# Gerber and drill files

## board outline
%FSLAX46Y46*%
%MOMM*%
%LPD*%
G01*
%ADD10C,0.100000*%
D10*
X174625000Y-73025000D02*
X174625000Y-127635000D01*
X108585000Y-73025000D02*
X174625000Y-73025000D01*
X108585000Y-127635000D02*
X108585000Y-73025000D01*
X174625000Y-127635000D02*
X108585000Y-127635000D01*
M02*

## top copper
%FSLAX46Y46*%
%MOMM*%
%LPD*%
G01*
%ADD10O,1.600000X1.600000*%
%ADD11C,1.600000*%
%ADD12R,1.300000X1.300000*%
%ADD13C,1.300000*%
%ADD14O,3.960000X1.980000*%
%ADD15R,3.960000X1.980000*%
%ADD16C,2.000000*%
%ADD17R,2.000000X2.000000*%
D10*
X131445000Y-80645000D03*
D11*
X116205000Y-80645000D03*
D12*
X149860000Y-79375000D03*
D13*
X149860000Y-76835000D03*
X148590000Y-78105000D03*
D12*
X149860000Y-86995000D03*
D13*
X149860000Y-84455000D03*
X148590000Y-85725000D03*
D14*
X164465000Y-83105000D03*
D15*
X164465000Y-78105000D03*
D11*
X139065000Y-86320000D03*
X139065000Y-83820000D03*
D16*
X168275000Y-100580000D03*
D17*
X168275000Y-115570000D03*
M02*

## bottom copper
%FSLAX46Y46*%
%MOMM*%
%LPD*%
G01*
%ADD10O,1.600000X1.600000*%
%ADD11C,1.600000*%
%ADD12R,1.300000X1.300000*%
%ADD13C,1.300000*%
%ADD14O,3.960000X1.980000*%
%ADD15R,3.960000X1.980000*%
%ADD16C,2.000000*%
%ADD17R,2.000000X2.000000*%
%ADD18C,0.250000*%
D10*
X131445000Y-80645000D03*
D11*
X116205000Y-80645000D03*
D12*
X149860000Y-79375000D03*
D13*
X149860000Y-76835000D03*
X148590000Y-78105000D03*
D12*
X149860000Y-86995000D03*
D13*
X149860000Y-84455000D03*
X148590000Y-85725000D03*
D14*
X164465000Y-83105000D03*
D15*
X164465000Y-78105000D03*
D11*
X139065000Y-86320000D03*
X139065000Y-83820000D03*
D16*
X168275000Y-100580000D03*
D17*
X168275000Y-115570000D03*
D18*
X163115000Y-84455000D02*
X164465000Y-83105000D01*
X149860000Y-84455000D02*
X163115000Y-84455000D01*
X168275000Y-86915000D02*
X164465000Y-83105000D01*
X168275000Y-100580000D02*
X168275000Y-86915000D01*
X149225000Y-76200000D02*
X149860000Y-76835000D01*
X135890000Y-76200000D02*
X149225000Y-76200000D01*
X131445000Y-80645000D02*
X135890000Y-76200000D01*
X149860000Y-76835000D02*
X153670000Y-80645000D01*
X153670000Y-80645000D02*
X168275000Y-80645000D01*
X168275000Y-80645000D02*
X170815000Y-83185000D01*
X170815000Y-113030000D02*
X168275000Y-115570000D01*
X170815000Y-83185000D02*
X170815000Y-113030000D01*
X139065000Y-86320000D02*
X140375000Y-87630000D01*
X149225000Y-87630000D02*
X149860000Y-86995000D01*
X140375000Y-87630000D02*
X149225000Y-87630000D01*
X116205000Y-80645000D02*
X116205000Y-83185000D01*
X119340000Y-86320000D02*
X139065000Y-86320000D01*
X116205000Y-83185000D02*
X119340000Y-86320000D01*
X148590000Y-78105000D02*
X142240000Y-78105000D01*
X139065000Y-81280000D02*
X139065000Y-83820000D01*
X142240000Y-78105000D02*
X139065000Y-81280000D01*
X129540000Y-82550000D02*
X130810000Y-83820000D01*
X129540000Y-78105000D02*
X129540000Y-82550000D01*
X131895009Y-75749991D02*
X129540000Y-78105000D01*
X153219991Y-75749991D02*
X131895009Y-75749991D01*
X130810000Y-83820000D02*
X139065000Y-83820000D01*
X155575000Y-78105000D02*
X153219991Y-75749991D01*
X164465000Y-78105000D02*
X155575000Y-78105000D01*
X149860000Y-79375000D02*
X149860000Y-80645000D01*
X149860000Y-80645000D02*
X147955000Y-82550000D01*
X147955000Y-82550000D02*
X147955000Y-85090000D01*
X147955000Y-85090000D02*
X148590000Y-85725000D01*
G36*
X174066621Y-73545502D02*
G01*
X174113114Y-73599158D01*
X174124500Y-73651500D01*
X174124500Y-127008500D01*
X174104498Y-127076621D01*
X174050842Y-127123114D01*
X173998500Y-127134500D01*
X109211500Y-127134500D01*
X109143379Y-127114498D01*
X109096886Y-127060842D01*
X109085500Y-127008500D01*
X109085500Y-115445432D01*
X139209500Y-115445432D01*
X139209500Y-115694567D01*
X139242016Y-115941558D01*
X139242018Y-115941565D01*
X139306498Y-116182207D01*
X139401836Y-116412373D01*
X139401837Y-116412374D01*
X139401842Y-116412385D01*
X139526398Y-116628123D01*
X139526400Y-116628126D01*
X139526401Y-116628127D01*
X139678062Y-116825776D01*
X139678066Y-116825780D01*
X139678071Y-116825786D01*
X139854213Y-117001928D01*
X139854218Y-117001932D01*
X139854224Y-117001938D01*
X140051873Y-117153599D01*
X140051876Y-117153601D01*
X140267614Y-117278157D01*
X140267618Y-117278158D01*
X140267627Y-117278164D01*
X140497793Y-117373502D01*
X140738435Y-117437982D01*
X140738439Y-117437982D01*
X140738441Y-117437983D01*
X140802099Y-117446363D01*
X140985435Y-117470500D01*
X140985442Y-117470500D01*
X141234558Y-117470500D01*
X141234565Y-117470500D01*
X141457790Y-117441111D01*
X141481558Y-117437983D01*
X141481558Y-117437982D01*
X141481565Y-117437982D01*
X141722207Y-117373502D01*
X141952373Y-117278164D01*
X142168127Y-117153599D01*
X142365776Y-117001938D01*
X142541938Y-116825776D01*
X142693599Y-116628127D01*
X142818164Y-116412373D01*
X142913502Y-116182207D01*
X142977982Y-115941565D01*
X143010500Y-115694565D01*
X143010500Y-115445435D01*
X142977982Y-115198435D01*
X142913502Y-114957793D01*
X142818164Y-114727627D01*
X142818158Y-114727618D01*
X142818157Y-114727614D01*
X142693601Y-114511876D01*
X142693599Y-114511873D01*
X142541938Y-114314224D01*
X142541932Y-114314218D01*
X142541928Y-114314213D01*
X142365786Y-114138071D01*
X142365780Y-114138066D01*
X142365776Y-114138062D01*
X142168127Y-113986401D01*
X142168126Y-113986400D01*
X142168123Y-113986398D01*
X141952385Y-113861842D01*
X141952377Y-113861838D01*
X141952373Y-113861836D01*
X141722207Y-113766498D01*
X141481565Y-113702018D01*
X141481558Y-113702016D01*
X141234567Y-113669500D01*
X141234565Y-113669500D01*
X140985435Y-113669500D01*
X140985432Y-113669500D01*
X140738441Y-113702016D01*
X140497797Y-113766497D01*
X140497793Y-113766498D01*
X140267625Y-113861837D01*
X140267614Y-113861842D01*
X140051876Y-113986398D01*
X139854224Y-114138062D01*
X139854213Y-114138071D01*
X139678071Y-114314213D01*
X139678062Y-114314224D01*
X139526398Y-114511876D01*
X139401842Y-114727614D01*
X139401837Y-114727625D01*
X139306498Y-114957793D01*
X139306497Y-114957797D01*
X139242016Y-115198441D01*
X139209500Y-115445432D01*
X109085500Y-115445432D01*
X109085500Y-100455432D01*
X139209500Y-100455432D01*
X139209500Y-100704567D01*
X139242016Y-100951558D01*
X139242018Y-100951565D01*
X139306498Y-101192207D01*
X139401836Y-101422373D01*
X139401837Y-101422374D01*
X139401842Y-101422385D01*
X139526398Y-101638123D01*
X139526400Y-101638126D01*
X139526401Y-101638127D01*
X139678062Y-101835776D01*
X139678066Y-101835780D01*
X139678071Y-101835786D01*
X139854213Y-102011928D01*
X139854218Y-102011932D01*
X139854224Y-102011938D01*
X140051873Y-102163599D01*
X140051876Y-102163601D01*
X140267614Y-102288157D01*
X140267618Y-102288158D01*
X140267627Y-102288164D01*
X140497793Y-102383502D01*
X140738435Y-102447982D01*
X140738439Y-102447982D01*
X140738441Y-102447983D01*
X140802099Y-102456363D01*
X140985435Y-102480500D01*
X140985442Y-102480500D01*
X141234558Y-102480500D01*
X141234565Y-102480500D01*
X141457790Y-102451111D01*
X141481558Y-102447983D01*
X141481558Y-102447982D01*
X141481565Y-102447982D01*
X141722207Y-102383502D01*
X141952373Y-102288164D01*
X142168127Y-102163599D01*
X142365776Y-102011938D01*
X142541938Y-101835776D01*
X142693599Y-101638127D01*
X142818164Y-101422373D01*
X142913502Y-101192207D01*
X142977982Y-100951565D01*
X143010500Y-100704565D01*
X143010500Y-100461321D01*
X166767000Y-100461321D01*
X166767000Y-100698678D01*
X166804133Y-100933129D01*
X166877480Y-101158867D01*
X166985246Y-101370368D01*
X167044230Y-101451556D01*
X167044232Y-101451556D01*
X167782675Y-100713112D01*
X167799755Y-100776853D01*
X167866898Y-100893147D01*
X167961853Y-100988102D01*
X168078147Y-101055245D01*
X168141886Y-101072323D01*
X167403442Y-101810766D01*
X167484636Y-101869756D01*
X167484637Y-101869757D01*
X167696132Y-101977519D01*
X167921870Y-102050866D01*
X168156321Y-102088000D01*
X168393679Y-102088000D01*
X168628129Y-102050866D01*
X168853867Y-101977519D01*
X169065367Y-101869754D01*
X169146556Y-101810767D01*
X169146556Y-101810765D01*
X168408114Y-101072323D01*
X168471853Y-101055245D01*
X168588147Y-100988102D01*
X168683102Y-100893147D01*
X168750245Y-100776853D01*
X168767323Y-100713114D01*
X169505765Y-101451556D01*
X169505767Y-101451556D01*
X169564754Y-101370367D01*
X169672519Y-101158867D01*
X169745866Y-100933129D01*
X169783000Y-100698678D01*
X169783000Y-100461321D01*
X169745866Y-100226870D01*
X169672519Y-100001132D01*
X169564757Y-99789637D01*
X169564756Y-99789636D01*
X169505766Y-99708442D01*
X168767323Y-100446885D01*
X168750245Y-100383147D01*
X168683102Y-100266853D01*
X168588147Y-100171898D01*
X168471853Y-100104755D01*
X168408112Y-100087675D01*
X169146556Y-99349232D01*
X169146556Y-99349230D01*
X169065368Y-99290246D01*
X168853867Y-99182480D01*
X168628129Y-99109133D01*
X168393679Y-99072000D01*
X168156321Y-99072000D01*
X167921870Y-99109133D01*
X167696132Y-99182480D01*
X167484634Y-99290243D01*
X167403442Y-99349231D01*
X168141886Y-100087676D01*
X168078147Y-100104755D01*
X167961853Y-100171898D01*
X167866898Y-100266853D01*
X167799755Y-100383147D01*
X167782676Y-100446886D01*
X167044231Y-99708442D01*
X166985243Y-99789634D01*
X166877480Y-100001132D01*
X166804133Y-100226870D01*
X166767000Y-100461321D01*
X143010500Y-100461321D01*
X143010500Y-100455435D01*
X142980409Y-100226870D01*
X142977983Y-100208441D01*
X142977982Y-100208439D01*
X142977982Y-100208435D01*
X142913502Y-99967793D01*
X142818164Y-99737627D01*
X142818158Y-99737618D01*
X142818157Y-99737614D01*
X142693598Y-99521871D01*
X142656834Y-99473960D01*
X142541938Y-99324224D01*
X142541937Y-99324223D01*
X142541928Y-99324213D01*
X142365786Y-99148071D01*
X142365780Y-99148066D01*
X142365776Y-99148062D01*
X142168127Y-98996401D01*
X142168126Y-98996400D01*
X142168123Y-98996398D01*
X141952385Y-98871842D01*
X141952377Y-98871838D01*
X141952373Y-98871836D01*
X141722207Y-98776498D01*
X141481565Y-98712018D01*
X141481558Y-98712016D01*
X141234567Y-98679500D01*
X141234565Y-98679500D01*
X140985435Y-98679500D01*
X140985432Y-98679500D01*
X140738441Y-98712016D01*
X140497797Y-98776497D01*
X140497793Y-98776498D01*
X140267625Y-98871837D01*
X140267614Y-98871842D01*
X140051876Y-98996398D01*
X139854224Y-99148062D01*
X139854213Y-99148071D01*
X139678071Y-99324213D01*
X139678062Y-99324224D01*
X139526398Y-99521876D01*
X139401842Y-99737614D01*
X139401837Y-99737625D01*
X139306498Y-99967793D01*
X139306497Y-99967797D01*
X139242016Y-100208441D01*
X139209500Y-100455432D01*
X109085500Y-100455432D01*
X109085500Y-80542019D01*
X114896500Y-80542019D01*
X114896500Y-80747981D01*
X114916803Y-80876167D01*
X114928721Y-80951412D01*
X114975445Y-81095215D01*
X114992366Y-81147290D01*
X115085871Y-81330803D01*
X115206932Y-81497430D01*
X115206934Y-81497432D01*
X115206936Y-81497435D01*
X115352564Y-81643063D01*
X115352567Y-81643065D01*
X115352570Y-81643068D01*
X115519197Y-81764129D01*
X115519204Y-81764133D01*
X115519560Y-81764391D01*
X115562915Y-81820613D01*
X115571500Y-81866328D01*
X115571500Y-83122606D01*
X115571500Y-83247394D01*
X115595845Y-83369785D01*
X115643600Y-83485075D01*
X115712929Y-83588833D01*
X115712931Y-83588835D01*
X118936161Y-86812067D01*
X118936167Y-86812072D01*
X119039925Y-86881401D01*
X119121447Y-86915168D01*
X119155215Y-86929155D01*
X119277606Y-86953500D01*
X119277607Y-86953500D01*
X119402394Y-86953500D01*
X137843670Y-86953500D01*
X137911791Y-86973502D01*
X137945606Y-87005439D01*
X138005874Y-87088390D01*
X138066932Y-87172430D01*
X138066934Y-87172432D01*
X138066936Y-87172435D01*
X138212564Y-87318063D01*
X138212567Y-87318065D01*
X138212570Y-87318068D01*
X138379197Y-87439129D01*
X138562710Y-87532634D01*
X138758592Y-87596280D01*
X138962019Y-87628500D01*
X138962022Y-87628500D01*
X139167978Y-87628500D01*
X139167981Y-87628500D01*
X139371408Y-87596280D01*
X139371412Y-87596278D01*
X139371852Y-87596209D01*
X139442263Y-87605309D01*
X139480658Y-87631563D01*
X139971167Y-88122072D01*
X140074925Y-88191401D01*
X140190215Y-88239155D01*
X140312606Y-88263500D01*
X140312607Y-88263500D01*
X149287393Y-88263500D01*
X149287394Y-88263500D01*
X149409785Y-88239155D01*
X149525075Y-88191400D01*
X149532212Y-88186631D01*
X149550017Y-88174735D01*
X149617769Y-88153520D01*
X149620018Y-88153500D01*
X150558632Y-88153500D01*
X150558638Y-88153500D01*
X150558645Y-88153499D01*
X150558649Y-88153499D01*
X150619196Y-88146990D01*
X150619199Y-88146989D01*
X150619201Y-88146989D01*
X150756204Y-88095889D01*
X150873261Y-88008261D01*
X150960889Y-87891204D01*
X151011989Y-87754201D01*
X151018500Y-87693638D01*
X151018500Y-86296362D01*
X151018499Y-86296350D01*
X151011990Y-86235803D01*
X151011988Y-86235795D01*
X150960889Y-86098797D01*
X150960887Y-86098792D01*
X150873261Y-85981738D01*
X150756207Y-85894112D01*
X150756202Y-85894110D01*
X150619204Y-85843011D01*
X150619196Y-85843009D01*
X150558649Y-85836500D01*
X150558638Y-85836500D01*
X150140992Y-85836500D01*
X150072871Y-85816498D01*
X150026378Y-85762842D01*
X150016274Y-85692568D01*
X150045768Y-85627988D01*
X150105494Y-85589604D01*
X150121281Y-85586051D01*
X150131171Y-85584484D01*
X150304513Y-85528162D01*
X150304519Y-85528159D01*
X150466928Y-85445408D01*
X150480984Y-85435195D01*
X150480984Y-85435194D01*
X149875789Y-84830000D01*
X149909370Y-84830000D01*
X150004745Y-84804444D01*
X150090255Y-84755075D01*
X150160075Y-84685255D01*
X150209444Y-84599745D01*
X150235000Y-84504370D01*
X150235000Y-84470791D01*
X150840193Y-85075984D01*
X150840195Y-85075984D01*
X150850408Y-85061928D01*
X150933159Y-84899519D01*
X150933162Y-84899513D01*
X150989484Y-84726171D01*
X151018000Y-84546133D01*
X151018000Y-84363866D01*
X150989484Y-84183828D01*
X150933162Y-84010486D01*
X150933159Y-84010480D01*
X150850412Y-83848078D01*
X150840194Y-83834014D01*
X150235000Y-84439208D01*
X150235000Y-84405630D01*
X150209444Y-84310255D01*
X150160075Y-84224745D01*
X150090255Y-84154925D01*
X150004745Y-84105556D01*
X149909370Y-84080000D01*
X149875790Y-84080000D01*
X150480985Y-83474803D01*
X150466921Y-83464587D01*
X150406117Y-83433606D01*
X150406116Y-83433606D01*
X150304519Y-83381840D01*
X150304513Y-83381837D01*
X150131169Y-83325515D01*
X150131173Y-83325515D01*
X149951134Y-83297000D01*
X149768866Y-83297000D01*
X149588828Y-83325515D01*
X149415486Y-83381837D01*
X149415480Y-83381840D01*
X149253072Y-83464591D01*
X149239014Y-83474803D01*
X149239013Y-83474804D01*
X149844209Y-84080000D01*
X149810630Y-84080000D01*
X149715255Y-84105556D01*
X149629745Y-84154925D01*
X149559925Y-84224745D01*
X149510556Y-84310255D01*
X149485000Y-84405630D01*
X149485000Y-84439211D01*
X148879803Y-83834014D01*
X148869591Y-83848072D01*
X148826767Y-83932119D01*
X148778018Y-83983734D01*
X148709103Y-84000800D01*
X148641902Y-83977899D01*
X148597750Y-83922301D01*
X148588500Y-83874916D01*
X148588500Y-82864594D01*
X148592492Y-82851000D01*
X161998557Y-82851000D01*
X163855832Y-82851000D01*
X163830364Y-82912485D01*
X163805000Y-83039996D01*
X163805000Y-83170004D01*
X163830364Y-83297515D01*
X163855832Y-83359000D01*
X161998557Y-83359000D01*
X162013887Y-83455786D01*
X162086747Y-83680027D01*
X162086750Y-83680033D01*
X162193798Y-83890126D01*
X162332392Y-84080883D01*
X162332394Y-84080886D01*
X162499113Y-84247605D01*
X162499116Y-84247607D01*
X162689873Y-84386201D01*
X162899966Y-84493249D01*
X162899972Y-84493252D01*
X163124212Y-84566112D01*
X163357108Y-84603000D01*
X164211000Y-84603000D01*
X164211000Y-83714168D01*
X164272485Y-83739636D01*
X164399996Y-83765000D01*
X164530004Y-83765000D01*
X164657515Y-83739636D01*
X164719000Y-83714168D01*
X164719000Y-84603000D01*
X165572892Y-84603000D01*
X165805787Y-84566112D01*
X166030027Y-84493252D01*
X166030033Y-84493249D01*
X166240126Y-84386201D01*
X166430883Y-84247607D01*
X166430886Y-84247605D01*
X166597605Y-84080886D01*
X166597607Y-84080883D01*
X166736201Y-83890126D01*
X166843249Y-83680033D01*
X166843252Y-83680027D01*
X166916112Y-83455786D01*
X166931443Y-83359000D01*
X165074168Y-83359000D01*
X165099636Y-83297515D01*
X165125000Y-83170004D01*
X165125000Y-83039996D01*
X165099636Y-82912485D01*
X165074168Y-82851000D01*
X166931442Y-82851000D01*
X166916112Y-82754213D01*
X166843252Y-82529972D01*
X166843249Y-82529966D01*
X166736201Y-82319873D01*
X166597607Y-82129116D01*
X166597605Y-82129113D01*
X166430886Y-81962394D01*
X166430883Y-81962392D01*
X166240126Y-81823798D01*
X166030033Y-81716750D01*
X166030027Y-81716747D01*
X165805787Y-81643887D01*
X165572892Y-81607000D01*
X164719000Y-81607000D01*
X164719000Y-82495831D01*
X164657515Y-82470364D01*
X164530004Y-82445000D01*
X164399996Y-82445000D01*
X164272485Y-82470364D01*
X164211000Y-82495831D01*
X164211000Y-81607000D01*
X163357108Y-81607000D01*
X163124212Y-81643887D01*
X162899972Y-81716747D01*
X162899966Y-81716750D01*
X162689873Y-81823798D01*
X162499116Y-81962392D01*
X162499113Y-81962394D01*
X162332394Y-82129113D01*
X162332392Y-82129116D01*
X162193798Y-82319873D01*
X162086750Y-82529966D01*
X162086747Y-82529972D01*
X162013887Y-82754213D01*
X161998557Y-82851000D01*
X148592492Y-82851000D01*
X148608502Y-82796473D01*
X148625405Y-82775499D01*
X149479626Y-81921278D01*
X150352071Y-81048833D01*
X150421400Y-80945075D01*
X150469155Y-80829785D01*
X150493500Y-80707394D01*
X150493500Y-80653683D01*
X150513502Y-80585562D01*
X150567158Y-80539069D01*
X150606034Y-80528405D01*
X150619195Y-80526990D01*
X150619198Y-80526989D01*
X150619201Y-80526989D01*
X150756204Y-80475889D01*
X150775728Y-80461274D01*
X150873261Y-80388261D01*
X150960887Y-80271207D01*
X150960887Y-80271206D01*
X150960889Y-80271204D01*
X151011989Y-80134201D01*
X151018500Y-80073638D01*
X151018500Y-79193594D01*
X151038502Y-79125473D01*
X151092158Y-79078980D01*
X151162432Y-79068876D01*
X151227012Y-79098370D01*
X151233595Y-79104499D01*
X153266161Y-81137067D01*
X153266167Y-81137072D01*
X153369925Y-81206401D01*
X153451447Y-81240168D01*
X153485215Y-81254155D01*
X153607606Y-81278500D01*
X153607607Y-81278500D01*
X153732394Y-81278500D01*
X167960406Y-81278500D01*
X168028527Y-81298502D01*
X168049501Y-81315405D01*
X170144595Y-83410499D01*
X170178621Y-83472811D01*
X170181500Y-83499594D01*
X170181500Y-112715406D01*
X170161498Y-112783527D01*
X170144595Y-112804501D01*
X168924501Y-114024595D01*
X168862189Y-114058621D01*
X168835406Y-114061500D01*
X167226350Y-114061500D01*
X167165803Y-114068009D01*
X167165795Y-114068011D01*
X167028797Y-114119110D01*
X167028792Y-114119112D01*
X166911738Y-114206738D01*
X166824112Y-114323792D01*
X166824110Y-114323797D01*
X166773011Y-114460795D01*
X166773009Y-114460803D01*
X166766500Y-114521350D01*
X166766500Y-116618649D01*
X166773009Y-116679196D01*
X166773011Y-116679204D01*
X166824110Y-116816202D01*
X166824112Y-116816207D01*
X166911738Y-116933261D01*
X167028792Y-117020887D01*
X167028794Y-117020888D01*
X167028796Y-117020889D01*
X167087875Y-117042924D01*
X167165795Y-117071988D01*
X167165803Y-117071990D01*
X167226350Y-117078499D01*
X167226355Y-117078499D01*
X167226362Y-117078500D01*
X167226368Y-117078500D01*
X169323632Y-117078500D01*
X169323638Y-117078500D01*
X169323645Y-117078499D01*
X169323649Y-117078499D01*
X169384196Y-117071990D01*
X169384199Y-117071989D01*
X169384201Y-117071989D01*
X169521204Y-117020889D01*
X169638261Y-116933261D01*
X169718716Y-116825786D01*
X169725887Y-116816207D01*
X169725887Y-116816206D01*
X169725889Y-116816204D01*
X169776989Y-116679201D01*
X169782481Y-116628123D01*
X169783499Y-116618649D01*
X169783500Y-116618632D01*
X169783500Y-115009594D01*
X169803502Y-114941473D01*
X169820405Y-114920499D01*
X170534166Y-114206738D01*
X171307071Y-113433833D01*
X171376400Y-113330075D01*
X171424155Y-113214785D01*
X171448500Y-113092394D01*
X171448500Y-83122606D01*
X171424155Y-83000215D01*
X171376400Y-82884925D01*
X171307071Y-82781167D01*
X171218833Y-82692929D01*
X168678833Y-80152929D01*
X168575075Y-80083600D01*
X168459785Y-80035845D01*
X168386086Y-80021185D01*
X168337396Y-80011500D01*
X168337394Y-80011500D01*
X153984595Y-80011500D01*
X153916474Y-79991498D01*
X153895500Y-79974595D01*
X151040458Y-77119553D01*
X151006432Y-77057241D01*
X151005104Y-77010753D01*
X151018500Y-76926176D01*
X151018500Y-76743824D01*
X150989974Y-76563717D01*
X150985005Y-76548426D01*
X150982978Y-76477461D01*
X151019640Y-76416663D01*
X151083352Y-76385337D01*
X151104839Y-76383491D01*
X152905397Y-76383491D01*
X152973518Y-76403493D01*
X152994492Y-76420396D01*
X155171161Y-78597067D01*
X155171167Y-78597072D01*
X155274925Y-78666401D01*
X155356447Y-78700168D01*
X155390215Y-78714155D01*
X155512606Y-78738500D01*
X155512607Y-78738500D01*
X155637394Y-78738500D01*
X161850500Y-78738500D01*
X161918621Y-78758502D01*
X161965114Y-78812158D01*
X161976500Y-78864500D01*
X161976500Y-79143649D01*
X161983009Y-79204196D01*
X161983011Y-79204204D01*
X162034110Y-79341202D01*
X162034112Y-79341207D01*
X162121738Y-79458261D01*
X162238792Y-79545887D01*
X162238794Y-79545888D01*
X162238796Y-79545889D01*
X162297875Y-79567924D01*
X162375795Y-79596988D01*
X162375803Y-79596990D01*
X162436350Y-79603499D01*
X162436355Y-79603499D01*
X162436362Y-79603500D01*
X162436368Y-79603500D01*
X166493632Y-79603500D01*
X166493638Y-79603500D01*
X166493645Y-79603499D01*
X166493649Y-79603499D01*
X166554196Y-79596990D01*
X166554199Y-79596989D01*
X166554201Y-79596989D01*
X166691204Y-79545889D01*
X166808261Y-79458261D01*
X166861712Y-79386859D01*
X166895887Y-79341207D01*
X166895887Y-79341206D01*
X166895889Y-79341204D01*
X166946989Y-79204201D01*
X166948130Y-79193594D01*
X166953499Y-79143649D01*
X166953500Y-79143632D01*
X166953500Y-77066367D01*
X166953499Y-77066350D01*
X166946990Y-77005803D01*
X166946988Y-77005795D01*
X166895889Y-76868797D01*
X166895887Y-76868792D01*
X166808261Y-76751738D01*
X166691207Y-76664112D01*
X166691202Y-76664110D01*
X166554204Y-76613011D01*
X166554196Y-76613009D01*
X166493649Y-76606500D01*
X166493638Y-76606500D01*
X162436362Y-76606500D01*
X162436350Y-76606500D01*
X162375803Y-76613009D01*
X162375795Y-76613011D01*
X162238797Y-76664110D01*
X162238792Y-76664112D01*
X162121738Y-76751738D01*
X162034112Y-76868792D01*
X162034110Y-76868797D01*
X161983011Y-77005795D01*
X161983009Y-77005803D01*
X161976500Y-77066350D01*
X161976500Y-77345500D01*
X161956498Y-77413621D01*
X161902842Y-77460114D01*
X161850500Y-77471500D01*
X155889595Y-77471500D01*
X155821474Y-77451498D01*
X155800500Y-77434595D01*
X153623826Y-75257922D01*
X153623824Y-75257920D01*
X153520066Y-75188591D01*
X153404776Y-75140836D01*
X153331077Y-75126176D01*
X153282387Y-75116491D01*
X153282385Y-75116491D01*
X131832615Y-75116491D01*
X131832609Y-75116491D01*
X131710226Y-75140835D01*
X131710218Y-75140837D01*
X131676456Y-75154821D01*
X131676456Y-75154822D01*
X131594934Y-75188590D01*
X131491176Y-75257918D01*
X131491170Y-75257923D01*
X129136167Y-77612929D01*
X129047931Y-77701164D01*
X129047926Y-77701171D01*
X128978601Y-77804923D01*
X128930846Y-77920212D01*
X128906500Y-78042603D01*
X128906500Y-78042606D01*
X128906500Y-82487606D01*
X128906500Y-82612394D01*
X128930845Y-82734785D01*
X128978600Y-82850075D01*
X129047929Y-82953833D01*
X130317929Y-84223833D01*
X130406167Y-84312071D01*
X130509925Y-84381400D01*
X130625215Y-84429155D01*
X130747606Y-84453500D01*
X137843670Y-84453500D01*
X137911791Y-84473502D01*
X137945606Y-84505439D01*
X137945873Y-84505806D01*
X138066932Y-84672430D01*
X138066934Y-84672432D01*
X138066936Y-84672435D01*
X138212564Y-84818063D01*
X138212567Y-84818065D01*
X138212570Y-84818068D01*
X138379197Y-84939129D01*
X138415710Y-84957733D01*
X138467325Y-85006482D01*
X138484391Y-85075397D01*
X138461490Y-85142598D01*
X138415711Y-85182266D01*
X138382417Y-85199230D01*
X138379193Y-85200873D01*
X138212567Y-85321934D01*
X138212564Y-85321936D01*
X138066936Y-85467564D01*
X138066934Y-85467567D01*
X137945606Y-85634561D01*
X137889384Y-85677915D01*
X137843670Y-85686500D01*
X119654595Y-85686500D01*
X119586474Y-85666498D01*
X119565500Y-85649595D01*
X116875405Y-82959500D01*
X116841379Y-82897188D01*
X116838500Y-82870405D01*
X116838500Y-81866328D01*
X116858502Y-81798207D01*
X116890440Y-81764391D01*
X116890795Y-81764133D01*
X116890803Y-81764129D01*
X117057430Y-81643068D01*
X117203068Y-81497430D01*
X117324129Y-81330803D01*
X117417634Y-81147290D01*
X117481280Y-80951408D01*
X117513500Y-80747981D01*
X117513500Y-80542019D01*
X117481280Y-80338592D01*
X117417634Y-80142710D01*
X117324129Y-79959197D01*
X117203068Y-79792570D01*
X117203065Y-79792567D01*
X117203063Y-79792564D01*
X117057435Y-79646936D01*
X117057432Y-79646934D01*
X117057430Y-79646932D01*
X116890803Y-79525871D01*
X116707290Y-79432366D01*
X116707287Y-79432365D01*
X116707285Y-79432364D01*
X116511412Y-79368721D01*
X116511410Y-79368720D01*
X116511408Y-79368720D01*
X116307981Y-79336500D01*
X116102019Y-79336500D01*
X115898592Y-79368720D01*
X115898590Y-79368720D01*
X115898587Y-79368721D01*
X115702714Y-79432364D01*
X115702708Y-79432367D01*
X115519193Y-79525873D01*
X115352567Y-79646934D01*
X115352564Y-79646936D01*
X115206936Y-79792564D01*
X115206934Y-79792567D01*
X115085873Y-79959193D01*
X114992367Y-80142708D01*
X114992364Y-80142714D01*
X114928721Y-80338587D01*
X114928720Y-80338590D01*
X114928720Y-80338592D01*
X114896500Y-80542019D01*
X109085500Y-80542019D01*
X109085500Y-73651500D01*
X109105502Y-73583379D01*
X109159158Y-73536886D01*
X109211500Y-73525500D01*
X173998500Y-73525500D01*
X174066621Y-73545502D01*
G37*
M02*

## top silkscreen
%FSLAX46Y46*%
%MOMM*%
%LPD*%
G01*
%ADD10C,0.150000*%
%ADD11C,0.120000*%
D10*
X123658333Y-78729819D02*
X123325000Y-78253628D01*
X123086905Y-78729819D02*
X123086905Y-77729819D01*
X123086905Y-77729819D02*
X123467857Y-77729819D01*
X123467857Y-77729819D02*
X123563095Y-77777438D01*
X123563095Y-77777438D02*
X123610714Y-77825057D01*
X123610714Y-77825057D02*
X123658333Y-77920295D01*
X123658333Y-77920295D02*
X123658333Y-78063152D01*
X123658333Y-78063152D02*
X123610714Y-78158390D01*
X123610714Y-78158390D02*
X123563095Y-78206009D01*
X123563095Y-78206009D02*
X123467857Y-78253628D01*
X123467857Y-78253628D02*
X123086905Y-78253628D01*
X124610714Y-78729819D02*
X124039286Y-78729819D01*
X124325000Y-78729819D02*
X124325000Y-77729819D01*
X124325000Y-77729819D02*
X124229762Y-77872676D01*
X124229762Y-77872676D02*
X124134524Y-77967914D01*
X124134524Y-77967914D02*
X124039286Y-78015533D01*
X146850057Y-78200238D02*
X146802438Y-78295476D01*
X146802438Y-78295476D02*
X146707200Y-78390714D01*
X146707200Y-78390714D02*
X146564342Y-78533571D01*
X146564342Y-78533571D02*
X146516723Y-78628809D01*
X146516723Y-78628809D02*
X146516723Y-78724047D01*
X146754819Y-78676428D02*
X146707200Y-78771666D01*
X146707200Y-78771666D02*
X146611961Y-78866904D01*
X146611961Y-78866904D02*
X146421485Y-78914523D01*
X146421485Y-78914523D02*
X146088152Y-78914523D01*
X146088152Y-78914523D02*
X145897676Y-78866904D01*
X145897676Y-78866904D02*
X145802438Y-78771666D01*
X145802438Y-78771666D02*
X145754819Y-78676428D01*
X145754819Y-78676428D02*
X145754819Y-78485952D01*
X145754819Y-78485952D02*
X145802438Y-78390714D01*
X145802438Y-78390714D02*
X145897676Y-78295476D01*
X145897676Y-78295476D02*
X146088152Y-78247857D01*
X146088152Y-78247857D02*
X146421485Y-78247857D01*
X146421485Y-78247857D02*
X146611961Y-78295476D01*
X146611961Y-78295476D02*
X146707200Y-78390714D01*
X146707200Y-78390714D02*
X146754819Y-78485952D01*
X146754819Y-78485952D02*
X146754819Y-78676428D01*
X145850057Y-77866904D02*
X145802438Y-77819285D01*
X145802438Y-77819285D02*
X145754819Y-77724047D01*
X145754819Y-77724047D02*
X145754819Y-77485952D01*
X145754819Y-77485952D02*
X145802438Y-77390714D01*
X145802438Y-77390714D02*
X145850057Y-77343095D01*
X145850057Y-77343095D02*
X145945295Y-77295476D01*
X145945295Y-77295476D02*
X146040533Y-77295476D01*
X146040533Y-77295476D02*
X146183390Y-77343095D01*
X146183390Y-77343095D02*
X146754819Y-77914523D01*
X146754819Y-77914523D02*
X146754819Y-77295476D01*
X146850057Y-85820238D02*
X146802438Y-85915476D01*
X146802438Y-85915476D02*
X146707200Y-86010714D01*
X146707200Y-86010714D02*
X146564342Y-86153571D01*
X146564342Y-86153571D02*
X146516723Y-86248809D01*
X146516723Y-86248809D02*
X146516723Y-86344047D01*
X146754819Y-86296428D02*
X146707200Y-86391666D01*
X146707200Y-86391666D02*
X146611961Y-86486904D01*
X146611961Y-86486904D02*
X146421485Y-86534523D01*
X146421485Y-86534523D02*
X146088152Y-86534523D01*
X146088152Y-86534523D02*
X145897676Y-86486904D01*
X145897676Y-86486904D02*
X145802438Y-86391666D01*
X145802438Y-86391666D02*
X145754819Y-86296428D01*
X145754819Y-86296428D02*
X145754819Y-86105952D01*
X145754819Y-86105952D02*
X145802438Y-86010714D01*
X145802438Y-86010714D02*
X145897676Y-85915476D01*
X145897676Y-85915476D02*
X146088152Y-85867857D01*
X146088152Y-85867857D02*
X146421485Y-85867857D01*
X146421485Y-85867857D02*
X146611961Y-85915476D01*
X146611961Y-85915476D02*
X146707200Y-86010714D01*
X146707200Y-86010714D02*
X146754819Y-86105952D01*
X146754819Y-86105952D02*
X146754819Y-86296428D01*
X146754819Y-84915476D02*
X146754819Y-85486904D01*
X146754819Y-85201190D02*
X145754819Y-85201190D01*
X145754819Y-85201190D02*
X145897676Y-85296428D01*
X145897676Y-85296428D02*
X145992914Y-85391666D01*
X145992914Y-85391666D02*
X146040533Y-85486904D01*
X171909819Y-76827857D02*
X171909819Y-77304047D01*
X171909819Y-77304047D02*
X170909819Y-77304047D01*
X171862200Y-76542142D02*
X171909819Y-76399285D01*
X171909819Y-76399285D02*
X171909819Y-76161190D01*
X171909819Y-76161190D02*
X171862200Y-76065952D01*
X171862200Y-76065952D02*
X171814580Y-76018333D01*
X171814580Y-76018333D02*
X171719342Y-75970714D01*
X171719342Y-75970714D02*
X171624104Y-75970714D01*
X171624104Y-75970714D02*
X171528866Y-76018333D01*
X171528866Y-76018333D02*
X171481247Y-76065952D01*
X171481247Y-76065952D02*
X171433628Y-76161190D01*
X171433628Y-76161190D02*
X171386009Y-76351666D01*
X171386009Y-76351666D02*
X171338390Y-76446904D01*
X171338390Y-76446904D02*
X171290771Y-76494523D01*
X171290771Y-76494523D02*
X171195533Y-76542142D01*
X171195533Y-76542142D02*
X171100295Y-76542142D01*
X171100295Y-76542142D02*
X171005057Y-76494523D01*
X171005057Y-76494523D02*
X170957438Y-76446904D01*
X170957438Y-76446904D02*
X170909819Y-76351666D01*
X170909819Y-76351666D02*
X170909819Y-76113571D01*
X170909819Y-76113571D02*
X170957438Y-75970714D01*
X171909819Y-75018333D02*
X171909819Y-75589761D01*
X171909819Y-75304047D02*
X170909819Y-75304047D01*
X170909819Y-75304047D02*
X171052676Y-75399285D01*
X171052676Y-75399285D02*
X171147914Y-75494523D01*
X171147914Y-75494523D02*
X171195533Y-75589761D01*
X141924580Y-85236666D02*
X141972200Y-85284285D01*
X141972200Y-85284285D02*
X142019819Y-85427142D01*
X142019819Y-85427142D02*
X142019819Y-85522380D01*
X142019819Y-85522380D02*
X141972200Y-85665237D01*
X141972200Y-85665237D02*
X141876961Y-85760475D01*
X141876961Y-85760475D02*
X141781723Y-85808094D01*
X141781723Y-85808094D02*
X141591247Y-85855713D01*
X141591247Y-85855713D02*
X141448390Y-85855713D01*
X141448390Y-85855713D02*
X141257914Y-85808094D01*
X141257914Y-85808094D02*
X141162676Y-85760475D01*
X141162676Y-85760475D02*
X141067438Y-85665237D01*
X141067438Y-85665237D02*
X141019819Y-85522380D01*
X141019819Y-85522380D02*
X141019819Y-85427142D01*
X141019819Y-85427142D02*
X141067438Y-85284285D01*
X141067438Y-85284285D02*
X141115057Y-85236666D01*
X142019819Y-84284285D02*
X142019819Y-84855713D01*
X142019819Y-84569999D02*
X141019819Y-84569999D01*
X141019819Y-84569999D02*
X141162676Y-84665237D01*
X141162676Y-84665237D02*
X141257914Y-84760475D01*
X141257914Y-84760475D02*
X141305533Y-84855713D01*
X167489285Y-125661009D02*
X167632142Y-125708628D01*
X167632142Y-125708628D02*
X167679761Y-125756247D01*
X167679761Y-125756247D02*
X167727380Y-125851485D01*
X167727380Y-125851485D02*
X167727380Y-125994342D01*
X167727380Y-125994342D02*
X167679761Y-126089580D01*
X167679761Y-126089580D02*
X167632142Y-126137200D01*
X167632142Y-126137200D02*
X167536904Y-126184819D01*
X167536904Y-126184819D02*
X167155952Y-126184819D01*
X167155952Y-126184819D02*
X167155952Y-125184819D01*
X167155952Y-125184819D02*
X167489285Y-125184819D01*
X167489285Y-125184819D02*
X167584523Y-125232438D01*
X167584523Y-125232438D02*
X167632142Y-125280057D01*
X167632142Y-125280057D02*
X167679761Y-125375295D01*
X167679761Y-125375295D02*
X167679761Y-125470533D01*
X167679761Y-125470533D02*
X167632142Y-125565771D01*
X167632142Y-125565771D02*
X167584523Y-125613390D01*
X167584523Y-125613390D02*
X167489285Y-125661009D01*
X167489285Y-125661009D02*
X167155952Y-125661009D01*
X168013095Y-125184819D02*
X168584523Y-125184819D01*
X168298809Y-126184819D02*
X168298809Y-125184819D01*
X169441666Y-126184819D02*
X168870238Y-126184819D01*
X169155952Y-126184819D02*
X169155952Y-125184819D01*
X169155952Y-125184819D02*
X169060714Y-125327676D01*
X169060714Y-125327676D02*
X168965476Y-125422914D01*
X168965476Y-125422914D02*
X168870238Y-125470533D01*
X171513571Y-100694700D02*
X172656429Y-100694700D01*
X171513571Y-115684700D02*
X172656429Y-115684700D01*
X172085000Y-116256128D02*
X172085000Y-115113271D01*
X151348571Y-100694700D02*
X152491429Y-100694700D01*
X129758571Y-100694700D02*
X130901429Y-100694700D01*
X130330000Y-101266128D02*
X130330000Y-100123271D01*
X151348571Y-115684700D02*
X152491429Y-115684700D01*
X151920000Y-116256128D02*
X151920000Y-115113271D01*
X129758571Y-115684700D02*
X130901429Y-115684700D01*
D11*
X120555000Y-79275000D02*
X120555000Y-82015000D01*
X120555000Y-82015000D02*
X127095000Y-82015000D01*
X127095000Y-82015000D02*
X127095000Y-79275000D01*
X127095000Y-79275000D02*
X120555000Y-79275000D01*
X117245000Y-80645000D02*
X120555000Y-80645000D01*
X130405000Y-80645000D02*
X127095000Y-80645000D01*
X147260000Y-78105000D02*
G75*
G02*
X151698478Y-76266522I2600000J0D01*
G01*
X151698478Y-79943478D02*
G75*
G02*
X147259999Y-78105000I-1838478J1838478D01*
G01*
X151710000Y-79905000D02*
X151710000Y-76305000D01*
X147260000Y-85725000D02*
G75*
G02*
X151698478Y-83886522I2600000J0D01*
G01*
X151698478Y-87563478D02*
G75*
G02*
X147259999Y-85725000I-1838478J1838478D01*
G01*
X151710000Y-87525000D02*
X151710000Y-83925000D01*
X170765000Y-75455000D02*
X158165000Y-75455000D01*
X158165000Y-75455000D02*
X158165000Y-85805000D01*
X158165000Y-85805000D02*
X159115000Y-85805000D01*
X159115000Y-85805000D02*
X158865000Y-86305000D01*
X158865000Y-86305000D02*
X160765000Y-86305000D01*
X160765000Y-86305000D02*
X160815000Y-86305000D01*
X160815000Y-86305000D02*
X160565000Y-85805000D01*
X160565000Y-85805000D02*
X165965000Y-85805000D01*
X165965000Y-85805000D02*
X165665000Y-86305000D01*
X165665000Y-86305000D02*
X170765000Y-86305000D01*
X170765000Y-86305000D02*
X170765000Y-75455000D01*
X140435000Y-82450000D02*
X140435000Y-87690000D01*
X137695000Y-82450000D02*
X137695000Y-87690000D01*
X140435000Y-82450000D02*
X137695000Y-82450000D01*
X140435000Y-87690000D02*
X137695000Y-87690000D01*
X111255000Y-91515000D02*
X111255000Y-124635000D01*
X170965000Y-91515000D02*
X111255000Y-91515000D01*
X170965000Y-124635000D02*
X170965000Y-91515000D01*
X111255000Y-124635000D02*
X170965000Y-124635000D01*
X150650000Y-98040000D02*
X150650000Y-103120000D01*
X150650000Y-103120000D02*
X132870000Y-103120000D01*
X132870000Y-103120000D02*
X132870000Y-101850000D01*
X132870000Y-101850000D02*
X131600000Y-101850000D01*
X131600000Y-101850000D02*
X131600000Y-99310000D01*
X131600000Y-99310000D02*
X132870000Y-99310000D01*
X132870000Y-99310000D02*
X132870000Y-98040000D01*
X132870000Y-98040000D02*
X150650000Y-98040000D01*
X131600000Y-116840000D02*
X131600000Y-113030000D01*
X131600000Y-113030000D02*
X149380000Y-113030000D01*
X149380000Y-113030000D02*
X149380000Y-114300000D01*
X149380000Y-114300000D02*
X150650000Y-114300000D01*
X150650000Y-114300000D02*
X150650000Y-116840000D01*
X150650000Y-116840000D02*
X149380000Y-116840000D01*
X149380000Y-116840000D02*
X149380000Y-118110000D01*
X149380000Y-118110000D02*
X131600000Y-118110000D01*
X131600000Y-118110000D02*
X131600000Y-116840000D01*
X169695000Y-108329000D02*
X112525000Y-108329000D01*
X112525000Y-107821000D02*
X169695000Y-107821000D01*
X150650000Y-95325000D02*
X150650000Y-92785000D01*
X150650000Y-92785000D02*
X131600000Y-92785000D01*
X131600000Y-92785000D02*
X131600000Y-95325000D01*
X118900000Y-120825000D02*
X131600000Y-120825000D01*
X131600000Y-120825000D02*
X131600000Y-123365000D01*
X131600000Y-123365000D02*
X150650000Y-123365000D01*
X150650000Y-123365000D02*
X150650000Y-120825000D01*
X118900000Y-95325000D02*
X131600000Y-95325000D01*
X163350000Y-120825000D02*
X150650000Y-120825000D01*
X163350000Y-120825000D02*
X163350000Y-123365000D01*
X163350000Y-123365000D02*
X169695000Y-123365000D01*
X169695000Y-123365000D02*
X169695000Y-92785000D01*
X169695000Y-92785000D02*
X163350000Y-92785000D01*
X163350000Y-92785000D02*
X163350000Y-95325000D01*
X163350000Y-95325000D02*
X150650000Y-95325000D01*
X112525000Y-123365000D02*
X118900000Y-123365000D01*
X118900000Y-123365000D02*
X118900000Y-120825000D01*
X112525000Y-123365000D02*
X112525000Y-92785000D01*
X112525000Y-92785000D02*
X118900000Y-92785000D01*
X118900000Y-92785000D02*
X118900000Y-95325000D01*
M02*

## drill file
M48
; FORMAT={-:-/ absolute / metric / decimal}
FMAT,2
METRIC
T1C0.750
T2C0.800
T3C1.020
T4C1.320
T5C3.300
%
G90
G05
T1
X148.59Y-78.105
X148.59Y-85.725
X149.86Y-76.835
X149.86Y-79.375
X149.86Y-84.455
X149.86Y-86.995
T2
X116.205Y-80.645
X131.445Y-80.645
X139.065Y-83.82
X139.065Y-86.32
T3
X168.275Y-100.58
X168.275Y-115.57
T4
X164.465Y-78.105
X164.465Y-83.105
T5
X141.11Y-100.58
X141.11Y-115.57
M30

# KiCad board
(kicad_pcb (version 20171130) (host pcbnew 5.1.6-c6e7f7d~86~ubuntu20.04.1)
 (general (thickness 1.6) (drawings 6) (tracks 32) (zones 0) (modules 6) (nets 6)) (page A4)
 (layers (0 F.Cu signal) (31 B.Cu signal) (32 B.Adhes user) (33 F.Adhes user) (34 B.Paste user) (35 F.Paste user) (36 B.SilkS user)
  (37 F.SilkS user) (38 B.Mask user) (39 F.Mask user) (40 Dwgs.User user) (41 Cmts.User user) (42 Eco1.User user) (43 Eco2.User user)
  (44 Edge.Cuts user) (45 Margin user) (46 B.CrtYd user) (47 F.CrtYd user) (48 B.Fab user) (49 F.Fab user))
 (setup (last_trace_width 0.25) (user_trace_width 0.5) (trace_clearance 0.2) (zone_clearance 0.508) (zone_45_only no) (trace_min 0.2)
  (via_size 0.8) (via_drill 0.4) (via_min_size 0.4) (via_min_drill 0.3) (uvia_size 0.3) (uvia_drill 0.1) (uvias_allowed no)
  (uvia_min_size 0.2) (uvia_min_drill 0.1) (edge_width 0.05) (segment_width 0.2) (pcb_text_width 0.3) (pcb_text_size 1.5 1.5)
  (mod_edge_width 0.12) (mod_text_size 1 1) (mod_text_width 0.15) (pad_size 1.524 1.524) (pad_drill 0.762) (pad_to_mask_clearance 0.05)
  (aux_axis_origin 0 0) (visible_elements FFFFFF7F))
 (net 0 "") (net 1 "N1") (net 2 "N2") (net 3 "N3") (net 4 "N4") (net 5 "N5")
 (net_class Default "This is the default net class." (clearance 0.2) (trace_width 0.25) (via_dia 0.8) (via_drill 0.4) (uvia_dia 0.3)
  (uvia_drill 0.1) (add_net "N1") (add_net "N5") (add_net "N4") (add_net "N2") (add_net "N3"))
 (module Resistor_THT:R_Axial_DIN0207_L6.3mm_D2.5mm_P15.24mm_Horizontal (layer F.Cu) (at 116.205 80.645)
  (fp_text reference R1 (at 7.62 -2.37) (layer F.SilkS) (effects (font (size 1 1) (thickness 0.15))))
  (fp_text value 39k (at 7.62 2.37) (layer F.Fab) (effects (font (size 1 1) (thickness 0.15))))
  (fp_line (start 4.35 -1.37) (end 4.35 1.37) (layer F.SilkS) (width 0.12))
  (fp_line (start 4.35 1.37) (end 10.89 1.37) (layer F.SilkS) (width 0.12))
  (fp_line (start 10.89 1.37) (end 10.89 -1.37) (layer F.SilkS) (width 0.12))
  (fp_line (start 10.89 -1.37) (end 4.35 -1.37) (layer F.SilkS) (width 0.12))
  (fp_line (start 1.04 0) (end 4.35 0) (layer F.SilkS) (width 0.12))
  (fp_line (start 14.2 0) (end 10.89 0) (layer F.SilkS) (width 0.12))
  (pad 2 thru_hole oval (at 15.24 0) (size 1.6 1.6) (drill 0.8) (layers *.Cu *.Mask) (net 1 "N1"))
  (pad 1 thru_hole circle (at 0 0) (size 1.6 1.6) (drill 0.8) (layers *.Cu *.Mask) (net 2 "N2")))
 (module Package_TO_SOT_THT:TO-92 (layer F.Cu) (at 149.86 79.375 90)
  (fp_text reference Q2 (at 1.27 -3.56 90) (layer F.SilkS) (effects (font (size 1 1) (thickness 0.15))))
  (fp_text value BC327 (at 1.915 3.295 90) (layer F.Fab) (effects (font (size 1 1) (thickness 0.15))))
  (fp_arc (start 1.27 0) (end 1.27 -2.6) (angle 135) (layer F.SilkS) (width 0.12))
  (fp_arc (start 1.27 0) (end 1.27 -2.6) (angle -135) (layer F.SilkS) (width 0.12))
  (fp_line (start -0.53 1.85) (end 3.07 1.85) (layer F.SilkS) (width 0.12))
  (pad 1 thru_hole rect (at 0 0 180) (size 1.3 1.3) (drill 0.75) (layers *.Cu *.Mask) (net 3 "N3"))
  (pad 3 thru_hole circle (at 2.54 0 180) (size 1.3 1.3) (drill 0.75) (layers *.Cu *.Mask) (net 1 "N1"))
  (pad 2 thru_hole circle (at 1.27 -1.27 180) (size 1.3 1.3) (drill 0.75) (layers *.Cu *.Mask) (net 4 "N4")))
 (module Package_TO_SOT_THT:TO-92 (layer F.Cu) (at 149.86 86.995 90)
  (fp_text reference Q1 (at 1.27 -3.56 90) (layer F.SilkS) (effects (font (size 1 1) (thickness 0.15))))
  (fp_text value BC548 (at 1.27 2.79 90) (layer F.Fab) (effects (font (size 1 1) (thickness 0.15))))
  (fp_arc (start 1.27 0) (end 1.27 -2.6) (angle 135) (layer F.SilkS) (width 0.12))
  (fp_arc (start 1.27 0) (end 1.27 -2.6) (angle -135) (layer F.SilkS) (width 0.12))
  (fp_line (start -0.53 1.85) (end 3.07 1.85) (layer F.SilkS) (width 0.12))
  (pad 1 thru_hole rect (at 0 0 180) (size 1.3 1.3) (drill 0.75) (layers *.Cu *.Mask) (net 2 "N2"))
  (pad 3 thru_hole circle (at 2.54 0 180) (size 1.3 1.3) (drill 0.75) (layers *.Cu *.Mask) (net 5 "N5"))
  (pad 2 thru_hole circle (at 1.27 -1.27 180) (size 1.3 1.3) (drill 0.75) (layers *.Cu *.Mask) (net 3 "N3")))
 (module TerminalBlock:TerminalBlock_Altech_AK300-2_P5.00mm (layer F.Cu) (at 164.465 78.105 270)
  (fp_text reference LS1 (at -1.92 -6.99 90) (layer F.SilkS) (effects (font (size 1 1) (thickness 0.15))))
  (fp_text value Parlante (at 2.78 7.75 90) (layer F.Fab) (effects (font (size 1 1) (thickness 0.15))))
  (fp_line (start -2.65 -6.3) (end -2.65 6.3) (layer F.SilkS) (width 0.12))
  (fp_line (start -2.65 6.3) (end 7.7 6.3) (layer F.SilkS) (width 0.12))
  (fp_line (start 7.7 6.3) (end 7.7 5.35) (layer F.SilkS) (width 0.12))
  (fp_line (start 7.7 5.35) (end 8.2 5.6) (layer F.SilkS) (width 0.12))
  (fp_line (start 8.2 5.6) (end 8.2 3.7) (layer F.SilkS) (width 0.12))
  (fp_line (start 8.2 3.7) (end 8.2 3.65) (layer F.SilkS) (width 0.12))
  (fp_line (start 8.2 3.65) (end 7.7 3.9) (layer F.SilkS) (width 0.12))
  (fp_line (start 7.7 3.9) (end 7.7 -1.5) (layer F.SilkS) (width 0.12))
  (fp_line (start 7.7 -1.5) (end 8.2 -1.2) (layer F.SilkS) (width 0.12))
  (fp_line (start 8.2 -1.2) (end 8.2 -6.3) (layer F.SilkS) (width 0.12))
  (fp_line (start 8.2 -6.3) (end -2.65 -6.3) (layer F.SilkS) (width 0.12))
  (pad 2 thru_hole oval (at 5 0 270) (size 1.98 3.96) (drill 1.32) (layers *.Cu *.Mask) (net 5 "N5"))
  (pad 1 thru_hole rect (at 0 0 270) (size 1.98 3.96) (drill 1.32) (layers *.Cu *.Mask) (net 4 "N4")))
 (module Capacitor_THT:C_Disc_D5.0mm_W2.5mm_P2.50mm (layer F.Cu) (at 139.065 83.82 270)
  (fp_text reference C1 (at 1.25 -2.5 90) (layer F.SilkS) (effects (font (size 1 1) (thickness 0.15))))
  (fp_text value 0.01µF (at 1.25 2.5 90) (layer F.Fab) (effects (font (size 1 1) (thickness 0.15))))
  (fp_line (start -1.37 -1.37) (end 3.87 -1.37) (layer F.SilkS) (width 0.12))
  (fp_line (start -1.37 1.37) (end 3.87 1.37) (layer F.SilkS) (width 0.12))
  (fp_line (start -1.37 -1.37) (end -1.37 1.37) (layer F.SilkS) (width 0.12))
  (fp_line (start 3.87 -1.37) (end 3.87 1.37) (layer F.SilkS) (width 0.12))
  (pad 2 thru_hole circle (at 2.5 0 270) (size 1.6 1.6) (drill 0.8) (layers *.Cu *.Mask) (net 2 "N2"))
  (pad 1 thru_hole circle (at 0 0 270) (size 1.6 1.6) (drill 0.8) (layers *.Cu *.Mask) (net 4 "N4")))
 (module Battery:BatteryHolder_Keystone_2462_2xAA (layer F.Cu) (at 168.275 115.57 180)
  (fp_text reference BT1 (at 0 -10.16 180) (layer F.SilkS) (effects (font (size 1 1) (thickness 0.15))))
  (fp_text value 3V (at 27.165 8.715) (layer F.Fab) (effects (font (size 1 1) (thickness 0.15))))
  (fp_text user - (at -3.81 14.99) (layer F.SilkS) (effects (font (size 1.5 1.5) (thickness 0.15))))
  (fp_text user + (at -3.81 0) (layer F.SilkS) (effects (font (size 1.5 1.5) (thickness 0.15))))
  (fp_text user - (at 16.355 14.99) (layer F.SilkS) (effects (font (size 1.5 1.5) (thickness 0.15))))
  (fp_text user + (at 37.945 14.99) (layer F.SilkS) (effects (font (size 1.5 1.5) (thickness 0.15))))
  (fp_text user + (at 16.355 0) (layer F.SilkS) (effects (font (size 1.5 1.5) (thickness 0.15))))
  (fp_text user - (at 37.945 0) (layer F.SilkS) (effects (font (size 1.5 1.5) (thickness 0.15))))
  (fp_line (start 57.02 24.055) (end 57.02 -9.065) (layer F.SilkS) (width 0.12))
  (fp_line (start -2.69 24.055) (end 57.02 24.055) (layer F.SilkS) (width 0.12))
  (fp_line (start -2.69 -9.065) (end -2.69 24.055) (layer F.SilkS) (width 0.12))
  (fp_line (start 57.02 -9.065) (end -2.69 -9.065) (layer F.SilkS) (width 0.12))
  (fp_line (start 17.625 17.53) (end 17.625 12.45) (layer F.SilkS) (width 0.12))
  (fp_line (start 17.625 12.45) (end 35.405 12.45) (layer F.SilkS) (width 0.12))
  (fp_line (start 35.405 12.45) (end 35.405 13.72) (layer F.SilkS) (width 0.12))
  (fp_line (start 35.405 13.72) (end 36.675 13.72) (layer F.SilkS) (width 0.12))
  (fp_line (start 36.675 13.72) (end 36.675 16.26) (layer F.SilkS) (width 0.12))
  (fp_line (start 36.675 16.26) (end 35.405 16.26) (layer F.SilkS) (width 0.12))
  (fp_line (start 35.405 16.26) (end 35.405 17.53) (layer F.SilkS) (width 0.12))
  (fp_line (start 35.405 17.53) (end 17.625 17.53) (layer F.SilkS) (width 0.12))
  (fp_line (start 36.675 -1.27) (end 36.675 2.54) (layer F.SilkS) (width 0.12))
  (fp_line (start 36.675 2.54) (end 18.895 2.54) (layer F.SilkS) (width 0.12))
  (fp_line (start 18.895 2.54) (end 18.895 1.27) (layer F.SilkS) (width 0.12))
  (fp_line (start 18.895 1.27) (end 17.625 1.27) (layer F.SilkS) (width 0.12))
  (fp_line (start 17.625 1.27) (end 17.625 -1.27) (layer F.SilkS) (width 0.12))
  (fp_line (start 17.625 -1.27) (end 18.895 -1.27) (layer F.SilkS) (width 0.12))
  (fp_line (start 18.895 -1.27) (end 18.895 -2.54) (layer F.SilkS) (width 0.12))
  (fp_line (start 18.895 -2.54) (end 36.675 -2.54) (layer F.SilkS) (width 0.12))
  (fp_line (start 36.675 -2.54) (end 36.675 -1.27) (layer F.SilkS) (width 0.12))
  (fp_line (start -1.42 7.241) (end 55.75 7.241) (layer F.SilkS) (width 0.12))
  (fp_line (start 55.75 7.749) (end -1.42 7.749) (layer F.SilkS) (width 0.12))
  (fp_line (start 17.625 20.245) (end 17.625 22.785) (layer F.SilkS) (width 0.12))
  (fp_line (start 17.625 22.785) (end 36.675 22.785) (layer F.SilkS) (width 0.12))
  (fp_line (start 36.675 22.785) (end 36.675 20.245) (layer F.SilkS) (width 0.12))
  (fp_line (start 49.375 -5.255) (end 36.675 -5.255) (layer F.SilkS) (width 0.12))
  (fp_line (start 36.675 -5.255) (end 36.675 -7.795) (layer F.SilkS) (width 0.12))
  (fp_line (start 36.675 -7.795) (end 17.625 -7.795) (layer F.SilkS) (width 0.12))
  (fp_line (start 17.625 -7.795) (end 17.625 -5.255) (layer F.SilkS) (width 0.12))
  (fp_line (start 49.375 20.245) (end 36.675 20.245) (layer F.SilkS) (width 0.12))
  (fp_line (start 4.925 -5.255) (end 17.625 -5.255) (layer F.SilkS) (width 0.12))
  (fp_line (start 4.925 -5.255) (end 4.925 -7.795) (layer F.SilkS) (width 0.12))
  (fp_line (start 4.925 -7.795) (end -1.42 -7.795) (layer F.SilkS) (width 0.12))
  (fp_line (start -1.42 -7.795) (end -1.42 22.785) (layer F.SilkS) (width 0.12))
  (fp_line (start -1.42 22.785) (end 4.925 22.785) (layer F.SilkS) (width 0.12))
  (fp_line (start 4.925 22.785) (end 4.925 20.245) (layer F.SilkS) (width 0.12))
  (fp_line (start 4.925 20.245) (end 17.625 20.245) (layer F.SilkS) (width 0.12))
  (fp_line (start 55.75 -7.795) (end 49.375 -7.795) (layer F.SilkS) (width 0.12))
  (fp_line (start 49.375 -7.795) (end 49.375 -5.255) (layer F.SilkS) (width 0.12))
  (fp_line (start 55.75 -7.795) (end 55.75 22.785) (layer F.SilkS) (width 0.12))
  (fp_line (start 55.75 22.785) (end 49.375 22.785) (layer F.SilkS) (width 0.12))
  (fp_line (start 49.375 22.785) (end 49.375 20.245) (layer F.SilkS) (width 0.12))
  (pad "" np_thru_hole circle (at 27.165 0 180) (size 3.3 3.3) (drill 3.3) (layers *.Cu *.Mask))
  (pad "" np_thru_hole circle (at 27.165 14.99 180) (size 3.3 3.3) (drill 3.3) (layers *.Cu *.Mask))
  (pad 2 thru_hole circle (at 0 14.99 180) (size 2 2) (drill 1.02) (layers *.Cu *.Mask) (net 5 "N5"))
  (pad 1 thru_hole rect (at 0 0 180) (size 2 2) (drill 1.02) (layers *.Cu *.Mask) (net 1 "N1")))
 (gr_line (start 174.625 73.025) (end 174.625 127.635) (layer Edge.Cuts) (width 0.1))
 (gr_line (start 108.585 73.025) (end 174.625 73.025) (layer Edge.Cuts) (width 0.1))
 (gr_line (start 108.585 127.635) (end 108.585 73.025) (layer Edge.Cuts) (width 0.1))
 (gr_line (start 174.625 127.635) (end 108.585 127.635) (layer Edge.Cuts) (width 0.1))
 (segment (start 163.115 84.455) (end 164.465 83.105) (width 0.25) (layer B.Cu) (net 5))
 (segment (start 149.86 84.455) (end 163.115 84.455) (width 0.25) (layer B.Cu) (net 5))
 (segment (start 168.275 86.915) (end 164.465 83.105) (width 0.25) (layer B.Cu) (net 5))
 (segment (start 168.275 100.58) (end 168.275 86.915) (width 0.25) (layer B.Cu) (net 5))
 (segment (start 149.225 76.2) (end 149.86 76.835) (width 0.25) (layer B.Cu) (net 1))
 (segment (start 135.89 76.2) (end 149.225 76.2) (width 0.25) (layer B.Cu) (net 1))
 (segment (start 131.445 80.645) (end 135.89 76.2) (width 0.25) (layer B.Cu) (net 1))
 (segment (start 149.86 76.835) (end 153.67 80.645) (width 0.25) (layer B.Cu) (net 1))
 (segment (start 153.67 80.645) (end 168.275 80.645) (width 0.25) (layer B.Cu) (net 1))
 (segment (start 168.275 80.645) (end 170.815 83.185) (width 0.25) (layer B.Cu) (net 1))
 (segment (start 170.815 113.03) (end 168.275 115.57) (width 0.25) (layer B.Cu) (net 1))
 (segment (start 170.815 83.185) (end 170.815 113.03) (width 0.25) (layer B.Cu) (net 1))
 (segment (start 139.065 86.32) (end 140.375 87.63) (width 0.25) (layer B.Cu) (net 2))
 (segment (start 149.225 87.63) (end 149.86 86.995) (width 0.25) (layer B.Cu) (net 2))
 (segment (start 140.375 87.63) (end 149.225 87.63) (width 0.25) (layer B.Cu) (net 2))
 (segment (start 116.205 80.645) (end 116.205 83.185) (width 0.25) (layer B.Cu) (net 2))
 (segment (start 119.34 86.32) (end 139.065 86.32) (width 0.25) (layer B.Cu) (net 2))
 (segment (start 116.205 83.185) (end 119.34 86.32) (width 0.25) (layer B.Cu) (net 2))
 (segment (start 148.59 78.105) (end 142.24 78.105) (width 0.25) (layer B.Cu) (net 4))
 (segment (start 139.065 81.28) (end 139.065 83.82) (width 0.25) (layer B.Cu) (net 4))
 (segment (start 142.24 78.105) (end 139.065 81.28) (width 0.25) (layer B.Cu) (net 4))
 (segment (start 129.54 82.55) (end 130.81 83.82) (width 0.25) (layer B.Cu) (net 4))
 (segment (start 129.54 78.105) (end 129.54 82.55) (width 0.25) (layer B.Cu) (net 4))
 (segment (start 131.895009 75.749991) (end 129.54 78.105) (width 0.25) (layer B.Cu) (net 4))
 (segment (start 153.219991 75.749991) (end 131.895009 75.749991) (width 0.25) (layer B.Cu) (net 4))
 (segment (start 130.81 83.82) (end 139.065 83.82) (width 0.25) (layer B.Cu) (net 4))
 (segment (start 155.575 78.105) (end 153.219991 75.749991) (width 0.25) (layer B.Cu) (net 4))
 (segment (start 164.465 78.105) (end 155.575 78.105) (width 0.25) (layer B.Cu) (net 4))
 (segment (start 149.86 79.375) (end 149.86 80.645) (width 0.25) (layer B.Cu) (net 3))
 (segment (start 149.86 80.645) (end 147.955 82.55) (width 0.25) (layer B.Cu) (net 3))
 (segment (start 147.955 82.55) (end 147.955 85.09) (width 0.25) (layer B.Cu) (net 3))
 (segment (start 147.955 85.09) (end 148.59 85.725) (width 0.25) (layer B.Cu) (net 3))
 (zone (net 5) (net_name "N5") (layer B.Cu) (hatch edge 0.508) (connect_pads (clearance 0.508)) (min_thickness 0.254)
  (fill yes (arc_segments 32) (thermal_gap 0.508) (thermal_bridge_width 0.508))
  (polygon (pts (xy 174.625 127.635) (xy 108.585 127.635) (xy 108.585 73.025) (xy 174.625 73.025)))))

